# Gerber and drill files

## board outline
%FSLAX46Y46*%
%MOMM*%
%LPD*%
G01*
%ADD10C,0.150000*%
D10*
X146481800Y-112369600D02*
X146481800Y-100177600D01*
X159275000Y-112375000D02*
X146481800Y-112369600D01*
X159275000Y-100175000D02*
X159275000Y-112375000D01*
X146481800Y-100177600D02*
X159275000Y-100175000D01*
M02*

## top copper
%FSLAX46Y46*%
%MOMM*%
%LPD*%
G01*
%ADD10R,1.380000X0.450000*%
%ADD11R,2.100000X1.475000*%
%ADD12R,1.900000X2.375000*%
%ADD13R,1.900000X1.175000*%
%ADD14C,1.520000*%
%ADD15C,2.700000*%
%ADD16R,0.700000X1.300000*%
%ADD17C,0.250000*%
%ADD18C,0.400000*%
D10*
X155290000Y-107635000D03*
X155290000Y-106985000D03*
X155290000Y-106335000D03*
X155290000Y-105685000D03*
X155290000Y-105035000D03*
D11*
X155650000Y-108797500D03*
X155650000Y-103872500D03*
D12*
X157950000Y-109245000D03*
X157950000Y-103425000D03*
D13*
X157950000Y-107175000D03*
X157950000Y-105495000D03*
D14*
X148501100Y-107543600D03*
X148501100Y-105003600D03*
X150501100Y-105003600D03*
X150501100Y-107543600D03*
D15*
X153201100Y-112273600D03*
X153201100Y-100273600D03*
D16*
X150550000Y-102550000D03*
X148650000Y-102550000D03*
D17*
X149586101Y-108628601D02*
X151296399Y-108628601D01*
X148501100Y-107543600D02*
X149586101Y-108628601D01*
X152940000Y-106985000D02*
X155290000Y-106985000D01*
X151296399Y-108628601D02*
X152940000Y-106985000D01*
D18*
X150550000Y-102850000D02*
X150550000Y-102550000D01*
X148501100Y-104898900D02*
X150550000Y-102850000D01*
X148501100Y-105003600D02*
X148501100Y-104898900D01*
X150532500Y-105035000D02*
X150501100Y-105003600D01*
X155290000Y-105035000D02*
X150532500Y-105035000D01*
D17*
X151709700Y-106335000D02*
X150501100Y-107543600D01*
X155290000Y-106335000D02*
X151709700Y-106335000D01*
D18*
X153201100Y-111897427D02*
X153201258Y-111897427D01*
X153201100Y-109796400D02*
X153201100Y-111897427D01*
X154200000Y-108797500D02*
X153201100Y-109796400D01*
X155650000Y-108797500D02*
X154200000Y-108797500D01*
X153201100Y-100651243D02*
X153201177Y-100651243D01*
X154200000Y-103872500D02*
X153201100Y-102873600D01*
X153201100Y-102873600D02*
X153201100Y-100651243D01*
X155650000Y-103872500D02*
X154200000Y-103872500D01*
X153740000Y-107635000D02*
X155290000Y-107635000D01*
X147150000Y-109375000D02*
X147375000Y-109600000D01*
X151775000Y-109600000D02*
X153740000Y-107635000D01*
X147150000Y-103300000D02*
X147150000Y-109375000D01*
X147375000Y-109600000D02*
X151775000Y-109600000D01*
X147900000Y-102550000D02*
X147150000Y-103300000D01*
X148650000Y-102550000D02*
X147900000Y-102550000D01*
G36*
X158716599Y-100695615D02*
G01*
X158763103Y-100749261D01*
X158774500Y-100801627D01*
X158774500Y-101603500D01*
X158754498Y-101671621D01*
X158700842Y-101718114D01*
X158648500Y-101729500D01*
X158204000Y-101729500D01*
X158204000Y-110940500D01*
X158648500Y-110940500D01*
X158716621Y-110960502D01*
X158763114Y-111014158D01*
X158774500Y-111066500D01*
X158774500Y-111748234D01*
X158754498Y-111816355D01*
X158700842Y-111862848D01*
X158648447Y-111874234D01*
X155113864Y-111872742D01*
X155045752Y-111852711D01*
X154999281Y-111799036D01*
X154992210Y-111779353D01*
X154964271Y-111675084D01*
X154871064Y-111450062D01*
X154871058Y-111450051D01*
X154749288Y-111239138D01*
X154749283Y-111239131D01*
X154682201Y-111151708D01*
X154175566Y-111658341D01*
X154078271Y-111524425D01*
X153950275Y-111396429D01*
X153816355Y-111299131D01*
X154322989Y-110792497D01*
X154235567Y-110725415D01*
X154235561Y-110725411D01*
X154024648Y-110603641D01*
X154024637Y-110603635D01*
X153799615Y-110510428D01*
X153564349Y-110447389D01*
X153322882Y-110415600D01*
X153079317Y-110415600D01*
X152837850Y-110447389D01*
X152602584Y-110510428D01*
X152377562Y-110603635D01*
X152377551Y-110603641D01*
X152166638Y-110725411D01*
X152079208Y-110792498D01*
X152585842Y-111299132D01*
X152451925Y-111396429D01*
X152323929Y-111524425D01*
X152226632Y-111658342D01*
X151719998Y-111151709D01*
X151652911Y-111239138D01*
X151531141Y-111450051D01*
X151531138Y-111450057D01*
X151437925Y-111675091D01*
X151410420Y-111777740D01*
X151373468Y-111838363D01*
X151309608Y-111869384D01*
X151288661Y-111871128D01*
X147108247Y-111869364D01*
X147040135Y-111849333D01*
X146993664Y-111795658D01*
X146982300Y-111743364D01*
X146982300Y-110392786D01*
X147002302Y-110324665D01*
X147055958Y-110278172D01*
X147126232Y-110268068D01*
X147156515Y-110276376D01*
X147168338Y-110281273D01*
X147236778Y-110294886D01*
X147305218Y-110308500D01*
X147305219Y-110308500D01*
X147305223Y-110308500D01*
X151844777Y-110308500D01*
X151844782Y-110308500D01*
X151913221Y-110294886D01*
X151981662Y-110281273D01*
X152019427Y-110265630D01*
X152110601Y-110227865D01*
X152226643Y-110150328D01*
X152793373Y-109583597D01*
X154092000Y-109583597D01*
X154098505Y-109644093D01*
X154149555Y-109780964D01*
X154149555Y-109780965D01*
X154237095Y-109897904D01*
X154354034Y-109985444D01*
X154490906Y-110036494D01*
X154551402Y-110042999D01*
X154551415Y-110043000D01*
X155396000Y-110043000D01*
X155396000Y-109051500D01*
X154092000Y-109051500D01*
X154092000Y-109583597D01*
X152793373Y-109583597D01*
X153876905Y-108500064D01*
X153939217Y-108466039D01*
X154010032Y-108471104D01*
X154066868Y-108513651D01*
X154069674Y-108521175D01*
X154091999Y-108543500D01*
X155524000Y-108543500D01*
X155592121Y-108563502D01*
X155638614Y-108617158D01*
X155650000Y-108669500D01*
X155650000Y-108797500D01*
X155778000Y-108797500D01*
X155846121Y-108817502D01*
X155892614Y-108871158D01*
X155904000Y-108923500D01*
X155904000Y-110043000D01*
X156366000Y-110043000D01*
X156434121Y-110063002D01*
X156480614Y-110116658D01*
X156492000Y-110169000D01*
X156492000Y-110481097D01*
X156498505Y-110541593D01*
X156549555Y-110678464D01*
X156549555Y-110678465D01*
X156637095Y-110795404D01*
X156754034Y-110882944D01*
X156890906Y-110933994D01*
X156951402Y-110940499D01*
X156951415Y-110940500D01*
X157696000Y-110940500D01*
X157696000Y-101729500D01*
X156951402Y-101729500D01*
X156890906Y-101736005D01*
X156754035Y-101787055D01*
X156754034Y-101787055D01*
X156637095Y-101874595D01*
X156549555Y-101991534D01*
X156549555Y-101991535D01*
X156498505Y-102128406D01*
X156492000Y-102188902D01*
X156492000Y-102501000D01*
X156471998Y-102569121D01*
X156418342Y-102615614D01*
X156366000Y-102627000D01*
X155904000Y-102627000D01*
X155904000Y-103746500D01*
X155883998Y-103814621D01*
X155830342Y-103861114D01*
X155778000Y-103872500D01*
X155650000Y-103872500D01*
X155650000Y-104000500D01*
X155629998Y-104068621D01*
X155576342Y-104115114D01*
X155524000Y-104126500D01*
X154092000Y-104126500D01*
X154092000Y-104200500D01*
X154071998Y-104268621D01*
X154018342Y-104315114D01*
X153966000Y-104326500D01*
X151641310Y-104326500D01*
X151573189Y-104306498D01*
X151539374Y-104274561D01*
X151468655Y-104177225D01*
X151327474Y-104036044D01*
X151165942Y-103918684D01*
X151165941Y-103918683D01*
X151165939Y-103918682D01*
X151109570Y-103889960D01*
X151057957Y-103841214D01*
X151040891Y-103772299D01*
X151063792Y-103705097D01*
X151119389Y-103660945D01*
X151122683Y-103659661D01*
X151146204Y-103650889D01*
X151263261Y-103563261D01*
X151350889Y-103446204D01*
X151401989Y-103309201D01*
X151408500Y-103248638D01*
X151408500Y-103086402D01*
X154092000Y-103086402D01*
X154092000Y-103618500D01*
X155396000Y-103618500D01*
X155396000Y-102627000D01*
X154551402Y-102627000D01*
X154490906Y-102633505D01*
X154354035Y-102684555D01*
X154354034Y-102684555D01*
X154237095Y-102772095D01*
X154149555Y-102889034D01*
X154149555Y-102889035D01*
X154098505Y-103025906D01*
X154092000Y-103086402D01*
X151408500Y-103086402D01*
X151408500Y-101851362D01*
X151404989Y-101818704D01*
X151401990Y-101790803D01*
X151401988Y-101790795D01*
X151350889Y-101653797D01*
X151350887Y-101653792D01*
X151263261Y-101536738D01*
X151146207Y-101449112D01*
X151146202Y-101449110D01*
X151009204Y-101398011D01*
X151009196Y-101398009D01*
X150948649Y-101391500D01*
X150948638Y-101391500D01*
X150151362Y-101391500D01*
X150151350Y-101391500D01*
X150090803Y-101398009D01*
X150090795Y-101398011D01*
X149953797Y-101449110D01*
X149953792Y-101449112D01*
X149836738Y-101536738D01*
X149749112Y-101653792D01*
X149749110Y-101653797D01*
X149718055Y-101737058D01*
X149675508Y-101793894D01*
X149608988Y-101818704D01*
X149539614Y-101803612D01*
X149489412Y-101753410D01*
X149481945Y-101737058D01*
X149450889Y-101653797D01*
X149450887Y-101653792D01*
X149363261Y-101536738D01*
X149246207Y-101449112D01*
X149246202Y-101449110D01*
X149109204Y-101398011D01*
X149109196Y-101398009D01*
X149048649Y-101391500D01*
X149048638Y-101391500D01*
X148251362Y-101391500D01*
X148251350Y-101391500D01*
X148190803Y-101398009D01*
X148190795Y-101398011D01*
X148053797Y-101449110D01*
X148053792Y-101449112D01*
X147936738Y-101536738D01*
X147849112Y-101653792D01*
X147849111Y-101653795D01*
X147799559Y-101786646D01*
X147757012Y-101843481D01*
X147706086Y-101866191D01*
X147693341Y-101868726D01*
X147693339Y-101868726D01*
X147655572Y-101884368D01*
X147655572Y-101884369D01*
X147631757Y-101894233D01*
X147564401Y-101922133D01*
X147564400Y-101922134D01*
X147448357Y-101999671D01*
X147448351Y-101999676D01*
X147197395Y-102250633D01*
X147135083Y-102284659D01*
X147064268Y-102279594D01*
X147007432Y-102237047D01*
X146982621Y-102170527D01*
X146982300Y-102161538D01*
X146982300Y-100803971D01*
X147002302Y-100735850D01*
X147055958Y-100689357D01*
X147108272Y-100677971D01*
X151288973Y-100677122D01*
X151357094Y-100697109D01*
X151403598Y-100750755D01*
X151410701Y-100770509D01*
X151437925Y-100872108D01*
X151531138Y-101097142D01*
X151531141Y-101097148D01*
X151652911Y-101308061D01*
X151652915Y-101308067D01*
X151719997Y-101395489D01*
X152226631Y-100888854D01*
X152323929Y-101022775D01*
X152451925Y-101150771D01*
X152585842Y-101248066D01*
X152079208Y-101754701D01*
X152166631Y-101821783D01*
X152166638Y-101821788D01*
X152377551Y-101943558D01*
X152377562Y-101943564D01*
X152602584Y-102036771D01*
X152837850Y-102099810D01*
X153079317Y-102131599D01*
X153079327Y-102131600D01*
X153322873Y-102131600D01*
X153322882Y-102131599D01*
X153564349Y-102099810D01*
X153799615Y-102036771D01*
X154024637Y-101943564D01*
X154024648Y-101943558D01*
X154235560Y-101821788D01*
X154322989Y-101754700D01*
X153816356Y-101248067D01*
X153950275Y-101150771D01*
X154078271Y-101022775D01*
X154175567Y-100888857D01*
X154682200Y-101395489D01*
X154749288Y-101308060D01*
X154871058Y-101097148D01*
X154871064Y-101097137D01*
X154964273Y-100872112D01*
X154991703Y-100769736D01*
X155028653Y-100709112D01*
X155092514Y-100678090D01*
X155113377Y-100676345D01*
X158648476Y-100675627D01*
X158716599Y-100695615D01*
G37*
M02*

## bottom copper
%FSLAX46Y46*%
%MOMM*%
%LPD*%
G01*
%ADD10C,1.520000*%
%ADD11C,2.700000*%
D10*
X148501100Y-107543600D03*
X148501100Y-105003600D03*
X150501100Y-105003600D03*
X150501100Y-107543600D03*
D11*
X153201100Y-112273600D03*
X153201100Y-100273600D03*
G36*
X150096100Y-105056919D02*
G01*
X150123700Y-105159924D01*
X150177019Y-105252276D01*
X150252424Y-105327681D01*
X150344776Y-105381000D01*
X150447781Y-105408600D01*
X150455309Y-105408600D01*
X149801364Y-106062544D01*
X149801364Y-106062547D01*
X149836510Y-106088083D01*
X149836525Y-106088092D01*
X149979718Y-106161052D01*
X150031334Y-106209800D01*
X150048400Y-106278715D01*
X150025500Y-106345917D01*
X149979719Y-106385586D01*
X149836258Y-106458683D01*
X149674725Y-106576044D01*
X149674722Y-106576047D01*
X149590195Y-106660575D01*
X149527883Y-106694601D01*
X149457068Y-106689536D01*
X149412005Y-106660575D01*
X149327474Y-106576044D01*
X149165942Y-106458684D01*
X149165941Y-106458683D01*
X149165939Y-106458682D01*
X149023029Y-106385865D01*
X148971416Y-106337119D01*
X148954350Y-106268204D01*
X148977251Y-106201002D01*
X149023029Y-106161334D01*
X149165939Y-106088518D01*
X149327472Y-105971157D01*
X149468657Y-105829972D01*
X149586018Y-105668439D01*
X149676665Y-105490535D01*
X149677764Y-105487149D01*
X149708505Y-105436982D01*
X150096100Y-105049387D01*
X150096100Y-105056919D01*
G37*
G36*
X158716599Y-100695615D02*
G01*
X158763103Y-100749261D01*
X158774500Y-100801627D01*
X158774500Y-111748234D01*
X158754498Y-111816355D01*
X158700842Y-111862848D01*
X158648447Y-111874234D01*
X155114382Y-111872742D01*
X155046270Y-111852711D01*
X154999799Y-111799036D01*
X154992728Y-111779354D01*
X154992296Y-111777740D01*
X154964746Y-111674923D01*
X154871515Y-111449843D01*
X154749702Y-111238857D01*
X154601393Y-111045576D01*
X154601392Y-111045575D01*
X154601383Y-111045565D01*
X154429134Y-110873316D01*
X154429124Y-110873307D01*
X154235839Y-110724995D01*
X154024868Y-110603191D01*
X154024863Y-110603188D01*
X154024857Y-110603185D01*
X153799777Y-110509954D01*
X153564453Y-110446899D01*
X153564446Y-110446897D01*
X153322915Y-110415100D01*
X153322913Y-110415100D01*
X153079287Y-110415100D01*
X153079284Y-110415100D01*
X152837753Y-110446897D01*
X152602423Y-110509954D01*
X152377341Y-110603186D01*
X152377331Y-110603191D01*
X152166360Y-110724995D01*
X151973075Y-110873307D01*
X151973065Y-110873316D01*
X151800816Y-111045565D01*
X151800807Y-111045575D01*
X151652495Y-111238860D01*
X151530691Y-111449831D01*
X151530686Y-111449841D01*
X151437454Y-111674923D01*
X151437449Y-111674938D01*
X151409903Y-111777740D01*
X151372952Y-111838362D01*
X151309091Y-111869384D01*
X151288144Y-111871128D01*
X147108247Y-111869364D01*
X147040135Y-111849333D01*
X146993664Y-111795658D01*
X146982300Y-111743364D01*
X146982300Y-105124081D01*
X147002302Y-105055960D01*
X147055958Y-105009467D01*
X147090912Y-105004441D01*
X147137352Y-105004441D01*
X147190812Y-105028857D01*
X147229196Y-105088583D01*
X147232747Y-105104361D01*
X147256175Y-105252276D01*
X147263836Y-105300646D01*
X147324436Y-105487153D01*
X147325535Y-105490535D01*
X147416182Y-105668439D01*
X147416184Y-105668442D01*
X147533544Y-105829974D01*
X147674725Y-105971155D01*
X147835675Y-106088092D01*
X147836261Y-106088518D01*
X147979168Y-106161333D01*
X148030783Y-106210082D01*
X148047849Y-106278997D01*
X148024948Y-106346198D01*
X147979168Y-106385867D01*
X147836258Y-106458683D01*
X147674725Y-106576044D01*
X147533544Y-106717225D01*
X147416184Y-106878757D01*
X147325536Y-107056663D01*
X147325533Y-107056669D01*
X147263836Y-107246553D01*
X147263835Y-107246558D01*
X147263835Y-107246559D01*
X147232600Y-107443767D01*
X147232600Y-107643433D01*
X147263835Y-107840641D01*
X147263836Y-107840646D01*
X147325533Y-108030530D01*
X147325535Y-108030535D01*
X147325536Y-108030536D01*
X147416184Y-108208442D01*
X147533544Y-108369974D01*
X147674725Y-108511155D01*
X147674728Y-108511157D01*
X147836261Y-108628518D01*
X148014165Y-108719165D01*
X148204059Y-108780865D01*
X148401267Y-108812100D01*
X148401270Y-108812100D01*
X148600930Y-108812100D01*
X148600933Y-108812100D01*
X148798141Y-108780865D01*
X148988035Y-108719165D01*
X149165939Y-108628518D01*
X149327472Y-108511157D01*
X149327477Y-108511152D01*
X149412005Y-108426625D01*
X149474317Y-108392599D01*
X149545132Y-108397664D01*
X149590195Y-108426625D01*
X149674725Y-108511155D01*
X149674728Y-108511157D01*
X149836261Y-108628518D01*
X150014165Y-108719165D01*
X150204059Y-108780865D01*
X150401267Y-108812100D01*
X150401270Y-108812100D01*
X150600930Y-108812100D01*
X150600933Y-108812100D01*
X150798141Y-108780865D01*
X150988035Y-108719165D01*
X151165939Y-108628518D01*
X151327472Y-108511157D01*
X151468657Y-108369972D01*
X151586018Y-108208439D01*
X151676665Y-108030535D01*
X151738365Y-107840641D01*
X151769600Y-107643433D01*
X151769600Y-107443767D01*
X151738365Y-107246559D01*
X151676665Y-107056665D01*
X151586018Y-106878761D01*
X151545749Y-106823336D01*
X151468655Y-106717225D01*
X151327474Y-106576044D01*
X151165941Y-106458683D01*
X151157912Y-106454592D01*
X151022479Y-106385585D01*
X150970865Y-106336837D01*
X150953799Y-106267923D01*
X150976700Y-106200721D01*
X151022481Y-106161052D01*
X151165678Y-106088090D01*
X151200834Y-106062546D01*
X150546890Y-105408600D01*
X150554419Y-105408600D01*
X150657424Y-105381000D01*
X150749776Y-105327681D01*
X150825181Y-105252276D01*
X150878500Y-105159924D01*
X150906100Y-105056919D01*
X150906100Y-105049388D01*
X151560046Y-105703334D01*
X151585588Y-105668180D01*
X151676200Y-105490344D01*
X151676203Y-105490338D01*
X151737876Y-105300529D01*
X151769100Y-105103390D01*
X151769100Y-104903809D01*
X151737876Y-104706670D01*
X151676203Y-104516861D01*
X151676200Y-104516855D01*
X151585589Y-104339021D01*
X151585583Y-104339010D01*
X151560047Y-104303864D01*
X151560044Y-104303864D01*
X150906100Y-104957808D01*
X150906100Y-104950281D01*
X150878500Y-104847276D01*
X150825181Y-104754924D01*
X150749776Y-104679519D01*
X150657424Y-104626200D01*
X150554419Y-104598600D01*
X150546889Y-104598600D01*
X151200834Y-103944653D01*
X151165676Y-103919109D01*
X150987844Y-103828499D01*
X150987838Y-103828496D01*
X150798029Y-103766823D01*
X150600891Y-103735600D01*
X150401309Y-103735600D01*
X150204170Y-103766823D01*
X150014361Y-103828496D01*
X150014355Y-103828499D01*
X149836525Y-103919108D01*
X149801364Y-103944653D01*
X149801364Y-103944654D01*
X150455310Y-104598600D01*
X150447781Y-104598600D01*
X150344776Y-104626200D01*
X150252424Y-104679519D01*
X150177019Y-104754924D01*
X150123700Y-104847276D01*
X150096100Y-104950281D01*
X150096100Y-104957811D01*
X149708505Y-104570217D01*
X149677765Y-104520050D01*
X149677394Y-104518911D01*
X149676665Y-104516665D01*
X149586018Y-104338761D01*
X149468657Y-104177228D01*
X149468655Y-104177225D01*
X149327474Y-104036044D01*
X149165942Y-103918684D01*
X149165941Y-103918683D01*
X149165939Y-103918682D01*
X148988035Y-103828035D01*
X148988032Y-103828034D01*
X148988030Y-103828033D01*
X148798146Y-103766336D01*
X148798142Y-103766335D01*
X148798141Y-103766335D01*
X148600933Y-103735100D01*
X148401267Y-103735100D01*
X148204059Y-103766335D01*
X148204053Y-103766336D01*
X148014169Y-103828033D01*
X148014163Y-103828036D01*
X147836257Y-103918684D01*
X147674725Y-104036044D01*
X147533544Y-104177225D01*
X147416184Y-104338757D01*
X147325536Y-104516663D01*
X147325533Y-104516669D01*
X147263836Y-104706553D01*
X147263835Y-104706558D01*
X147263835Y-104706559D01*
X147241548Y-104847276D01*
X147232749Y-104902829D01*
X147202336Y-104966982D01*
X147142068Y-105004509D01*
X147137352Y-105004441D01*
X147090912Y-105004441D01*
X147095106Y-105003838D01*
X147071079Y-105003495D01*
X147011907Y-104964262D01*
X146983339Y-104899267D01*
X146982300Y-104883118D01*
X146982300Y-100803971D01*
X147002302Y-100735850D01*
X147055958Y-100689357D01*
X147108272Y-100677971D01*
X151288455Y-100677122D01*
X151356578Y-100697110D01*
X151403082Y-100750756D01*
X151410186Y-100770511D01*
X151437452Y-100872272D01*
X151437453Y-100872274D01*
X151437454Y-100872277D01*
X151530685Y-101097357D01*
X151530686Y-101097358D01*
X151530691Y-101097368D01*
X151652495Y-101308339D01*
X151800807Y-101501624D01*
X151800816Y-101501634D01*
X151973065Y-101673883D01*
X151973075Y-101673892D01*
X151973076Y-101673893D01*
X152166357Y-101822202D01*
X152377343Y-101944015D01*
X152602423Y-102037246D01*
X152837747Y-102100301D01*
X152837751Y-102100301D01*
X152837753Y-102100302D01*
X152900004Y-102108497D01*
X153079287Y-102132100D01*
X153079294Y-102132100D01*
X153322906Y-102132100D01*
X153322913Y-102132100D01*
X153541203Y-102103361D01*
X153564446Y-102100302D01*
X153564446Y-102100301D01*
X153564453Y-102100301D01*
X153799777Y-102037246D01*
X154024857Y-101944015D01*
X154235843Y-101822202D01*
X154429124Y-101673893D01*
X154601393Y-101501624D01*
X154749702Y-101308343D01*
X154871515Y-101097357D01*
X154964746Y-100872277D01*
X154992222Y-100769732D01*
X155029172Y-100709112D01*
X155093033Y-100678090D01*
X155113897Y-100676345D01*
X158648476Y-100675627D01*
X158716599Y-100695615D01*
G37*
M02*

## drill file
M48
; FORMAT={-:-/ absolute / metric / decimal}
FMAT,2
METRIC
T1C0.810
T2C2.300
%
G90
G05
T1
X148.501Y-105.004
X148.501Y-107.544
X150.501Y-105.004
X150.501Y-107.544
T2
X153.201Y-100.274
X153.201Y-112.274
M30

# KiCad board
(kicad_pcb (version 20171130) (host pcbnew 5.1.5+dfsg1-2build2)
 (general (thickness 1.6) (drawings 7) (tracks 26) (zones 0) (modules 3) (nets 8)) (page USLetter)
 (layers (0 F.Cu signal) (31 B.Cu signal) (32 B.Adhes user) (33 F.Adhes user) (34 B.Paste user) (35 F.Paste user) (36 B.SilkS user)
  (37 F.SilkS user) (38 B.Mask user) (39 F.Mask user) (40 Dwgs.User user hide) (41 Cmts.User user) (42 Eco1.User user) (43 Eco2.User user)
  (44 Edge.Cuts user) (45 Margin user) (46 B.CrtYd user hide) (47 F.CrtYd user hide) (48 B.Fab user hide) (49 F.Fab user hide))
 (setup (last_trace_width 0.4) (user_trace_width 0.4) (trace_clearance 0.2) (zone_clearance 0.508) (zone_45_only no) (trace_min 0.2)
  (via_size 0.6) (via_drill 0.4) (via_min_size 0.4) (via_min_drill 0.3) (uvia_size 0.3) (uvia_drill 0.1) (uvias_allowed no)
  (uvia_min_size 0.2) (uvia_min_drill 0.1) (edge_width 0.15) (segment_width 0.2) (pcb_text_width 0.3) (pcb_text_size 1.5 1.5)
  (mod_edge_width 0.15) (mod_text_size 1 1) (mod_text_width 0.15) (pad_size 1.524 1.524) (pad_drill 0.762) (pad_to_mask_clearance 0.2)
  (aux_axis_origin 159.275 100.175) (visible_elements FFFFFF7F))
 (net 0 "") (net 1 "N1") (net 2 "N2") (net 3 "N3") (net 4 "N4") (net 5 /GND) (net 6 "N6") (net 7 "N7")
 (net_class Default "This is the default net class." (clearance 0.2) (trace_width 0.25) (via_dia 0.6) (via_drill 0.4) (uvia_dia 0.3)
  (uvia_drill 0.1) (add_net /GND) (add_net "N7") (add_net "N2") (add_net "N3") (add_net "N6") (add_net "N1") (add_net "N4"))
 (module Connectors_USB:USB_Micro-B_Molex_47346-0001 (layer F.Cu) (at 157.95 106.335 90)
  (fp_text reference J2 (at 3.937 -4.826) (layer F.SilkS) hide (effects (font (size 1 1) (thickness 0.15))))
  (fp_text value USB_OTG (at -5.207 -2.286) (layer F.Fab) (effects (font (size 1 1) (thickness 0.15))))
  (pad 1 smd rect (at -1.3 -2.66 90) (size 0.45 1.38) (layers F.Cu F.Paste F.Mask) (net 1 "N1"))
  (pad 2 smd rect (at -0.65 -2.66 90) (size 0.45 1.38) (layers F.Cu F.Paste F.Mask) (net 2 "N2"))
  (pad 3 smd rect (at 0 -2.66 90) (size 0.45 1.38) (layers F.Cu F.Paste F.Mask) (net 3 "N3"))
  (pad 4 smd rect (at 0.65 -2.66 90) (size 0.45 1.38) (layers F.Cu F.Paste F.Mask) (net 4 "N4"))
  (pad 5 smd rect (at 1.3 -2.66 90) (size 0.45 1.38) (layers F.Cu F.Paste F.Mask) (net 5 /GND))
  (pad 6 smd rect (at -2.4625 -2.3 90) (size 1.475 2.1) (layers F.Cu F.Paste F.Mask) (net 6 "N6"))
  (pad 6 smd rect (at 2.4625 -2.3 90) (size 1.475 2.1) (layers F.Cu F.Paste F.Mask) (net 6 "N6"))
  (pad 6 smd rect (at -2.91 0 90) (size 2.375 1.9) (layers F.Cu F.Paste F.Mask) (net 6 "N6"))
  (pad 6 smd rect (at 2.91 0 90) (size 2.375 1.9) (layers F.Cu F.Paste F.Mask) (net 6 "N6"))
  (pad 6 smd rect (at -0.84 0 90) (size 1.175 1.9) (layers F.Cu F.Paste F.Mask) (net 6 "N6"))
  (pad 6 smd rect (at 0.84 0 90) (size 1.175 1.9) (layers F.Cu F.Paste F.Mask) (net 6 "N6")))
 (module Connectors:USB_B (layer F.Cu) (at 148.5011 105.0036)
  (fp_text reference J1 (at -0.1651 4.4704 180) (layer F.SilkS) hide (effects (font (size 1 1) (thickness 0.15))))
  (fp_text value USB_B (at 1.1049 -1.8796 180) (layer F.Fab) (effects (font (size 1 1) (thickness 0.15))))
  (pad 2 thru_hole circle (at 0 2.54 270) (size 1.52 1.52) (drill 0.81) (layers *.Cu *.Mask) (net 2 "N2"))
  (pad 1 thru_hole circle (at 0 0 270) (size 1.52 1.52) (drill 0.81) (layers *.Cu *.Mask) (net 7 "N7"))
  (pad 4 thru_hole circle (at 2 0 270) (size 1.52 1.52) (drill 0.81) (layers *.Cu *.Mask) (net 5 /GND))
  (pad 3 thru_hole circle (at 2 2.54 270) (size 1.52 1.52) (drill 0.81) (layers *.Cu *.Mask) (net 3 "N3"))
  (pad 5 thru_hole circle (at 4.7 7.27 270) (size 2.7 2.7) (drill 2.3) (layers *.Cu *.Mask) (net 6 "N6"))
  (pad 5 thru_hole circle (at 4.7 -4.73 270) (size 2.7 2.7) (drill 2.3) (layers *.Cu *.Mask) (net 6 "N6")))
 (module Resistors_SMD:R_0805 (layer F.Cu) (at 149.6 102.55 180)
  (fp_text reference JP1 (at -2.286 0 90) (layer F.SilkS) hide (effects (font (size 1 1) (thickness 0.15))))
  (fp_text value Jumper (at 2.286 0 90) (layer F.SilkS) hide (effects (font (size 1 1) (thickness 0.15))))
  (pad 1 smd rect (at -0.95 0 180) (size 0.7 1.3) (layers F.Cu F.Paste F.Mask) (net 7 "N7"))
  (pad 2 smd rect (at 0.95 0 180) (size 0.7 1.3) (layers F.Cu F.Paste F.Mask) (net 1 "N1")))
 (gr_line (start 146.4818 112.3696) (end 146.4818 100.1776) (angle 90) (layer Edge.Cuts) (width 0.15))
 (gr_line (start 159.275 112.375) (end 146.4818 112.3696) (angle 90) (layer Edge.Cuts) (width 0.15))
 (gr_line (start 159.275 100.175) (end 159.275 112.375) (angle 90) (layer Edge.Cuts) (width 0.15))
 (gr_line (start 146.4818 100.1776) (end 159.275 100.175) (angle 90) (layer Edge.Cuts) (width 0.15))
 (segment (start 149.586101 108.628601) (end 151.296399 108.628601) (width 0.25) (layer F.Cu) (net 2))
 (segment (start 148.5011 107.5436) (end 149.586101 108.628601) (width 0.25) (layer F.Cu) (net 2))
 (segment (start 152.94 106.985) (end 155.29 106.985) (width 0.25) (layer F.Cu) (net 2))
 (segment (start 151.296399 108.628601) (end 152.94 106.985) (width 0.25) (layer F.Cu) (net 2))
 (segment (start 150.55 102.85) (end 150.55 102.55) (width 0.4) (layer F.Cu) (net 7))
 (segment (start 148.5011 104.8989) (end 150.55 102.85) (width 0.4) (layer F.Cu) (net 7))
 (segment (start 148.5011 105.0036) (end 148.5011 104.8989) (width 0.4) (layer F.Cu) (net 7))
 (segment (start 150.5325 105.035) (end 150.5011 105.0036) (width 0.4) (layer F.Cu) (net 5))
 (segment (start 155.29 105.035) (end 150.5325 105.035) (width 0.4) (layer F.Cu) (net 5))
 (segment (start 151.7097 106.335) (end 150.5011 107.5436) (width 0.25) (layer F.Cu) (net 3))
 (segment (start 155.29 106.335) (end 151.7097 106.335) (width 0.25) (layer F.Cu) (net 3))
 (segment (start 153.2011 111.897427) (end 153.201258 111.897427) (width 0.4) (layer F.Cu) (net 6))
 (segment (start 153.2011 109.7964) (end 153.2011 111.897427) (width 0.4) (layer F.Cu) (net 6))
 (segment (start 154.2 108.7975) (end 153.2011 109.7964) (width 0.4) (layer F.Cu) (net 6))
 (segment (start 155.65 108.7975) (end 154.2 108.7975) (width 0.4) (layer F.Cu) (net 6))
 (segment (start 153.2011 100.651243) (end 153.201177 100.651243) (width 0.4) (layer F.Cu) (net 6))
 (segment (start 154.2 103.8725) (end 153.2011 102.8736) (width 0.4) (layer F.Cu) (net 6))
 (segment (start 153.2011 102.8736) (end 153.2011 100.651243) (width 0.4) (layer F.Cu) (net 6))
 (segment (start 155.65 103.8725) (end 154.2 103.8725) (width 0.4) (layer F.Cu) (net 6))
 (segment (start 153.74 107.635) (end 155.29 107.635) (width 0.4) (layer F.Cu) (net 1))
 (segment (start 147.15 109.375) (end 147.375 109.6) (width 0.4) (layer F.Cu) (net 1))
 (segment (start 151.775 109.6) (end 153.74 107.635) (width 0.4) (layer F.Cu) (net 1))
 (segment (start 147.15 103.3) (end 147.15 109.375) (width 0.4) (layer F.Cu) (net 1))
 (segment (start 147.375 109.6) (end 151.775 109.6) (width 0.4) (layer F.Cu) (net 1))
 (segment (start 147.9 102.55) (end 147.15 103.3) (width 0.4) (layer F.Cu) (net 1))
 (segment (start 148.65 102.55) (end 147.9 102.55) (width 0.4) (layer F.Cu) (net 1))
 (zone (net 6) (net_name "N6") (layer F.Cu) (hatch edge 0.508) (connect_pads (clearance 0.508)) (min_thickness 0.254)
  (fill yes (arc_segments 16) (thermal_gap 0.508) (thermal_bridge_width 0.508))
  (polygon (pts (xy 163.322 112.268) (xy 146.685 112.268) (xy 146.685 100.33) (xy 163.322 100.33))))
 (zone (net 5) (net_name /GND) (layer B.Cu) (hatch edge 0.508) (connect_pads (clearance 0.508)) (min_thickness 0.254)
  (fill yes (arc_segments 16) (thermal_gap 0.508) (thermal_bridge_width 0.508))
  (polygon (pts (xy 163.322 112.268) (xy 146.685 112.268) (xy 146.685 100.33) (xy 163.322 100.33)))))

